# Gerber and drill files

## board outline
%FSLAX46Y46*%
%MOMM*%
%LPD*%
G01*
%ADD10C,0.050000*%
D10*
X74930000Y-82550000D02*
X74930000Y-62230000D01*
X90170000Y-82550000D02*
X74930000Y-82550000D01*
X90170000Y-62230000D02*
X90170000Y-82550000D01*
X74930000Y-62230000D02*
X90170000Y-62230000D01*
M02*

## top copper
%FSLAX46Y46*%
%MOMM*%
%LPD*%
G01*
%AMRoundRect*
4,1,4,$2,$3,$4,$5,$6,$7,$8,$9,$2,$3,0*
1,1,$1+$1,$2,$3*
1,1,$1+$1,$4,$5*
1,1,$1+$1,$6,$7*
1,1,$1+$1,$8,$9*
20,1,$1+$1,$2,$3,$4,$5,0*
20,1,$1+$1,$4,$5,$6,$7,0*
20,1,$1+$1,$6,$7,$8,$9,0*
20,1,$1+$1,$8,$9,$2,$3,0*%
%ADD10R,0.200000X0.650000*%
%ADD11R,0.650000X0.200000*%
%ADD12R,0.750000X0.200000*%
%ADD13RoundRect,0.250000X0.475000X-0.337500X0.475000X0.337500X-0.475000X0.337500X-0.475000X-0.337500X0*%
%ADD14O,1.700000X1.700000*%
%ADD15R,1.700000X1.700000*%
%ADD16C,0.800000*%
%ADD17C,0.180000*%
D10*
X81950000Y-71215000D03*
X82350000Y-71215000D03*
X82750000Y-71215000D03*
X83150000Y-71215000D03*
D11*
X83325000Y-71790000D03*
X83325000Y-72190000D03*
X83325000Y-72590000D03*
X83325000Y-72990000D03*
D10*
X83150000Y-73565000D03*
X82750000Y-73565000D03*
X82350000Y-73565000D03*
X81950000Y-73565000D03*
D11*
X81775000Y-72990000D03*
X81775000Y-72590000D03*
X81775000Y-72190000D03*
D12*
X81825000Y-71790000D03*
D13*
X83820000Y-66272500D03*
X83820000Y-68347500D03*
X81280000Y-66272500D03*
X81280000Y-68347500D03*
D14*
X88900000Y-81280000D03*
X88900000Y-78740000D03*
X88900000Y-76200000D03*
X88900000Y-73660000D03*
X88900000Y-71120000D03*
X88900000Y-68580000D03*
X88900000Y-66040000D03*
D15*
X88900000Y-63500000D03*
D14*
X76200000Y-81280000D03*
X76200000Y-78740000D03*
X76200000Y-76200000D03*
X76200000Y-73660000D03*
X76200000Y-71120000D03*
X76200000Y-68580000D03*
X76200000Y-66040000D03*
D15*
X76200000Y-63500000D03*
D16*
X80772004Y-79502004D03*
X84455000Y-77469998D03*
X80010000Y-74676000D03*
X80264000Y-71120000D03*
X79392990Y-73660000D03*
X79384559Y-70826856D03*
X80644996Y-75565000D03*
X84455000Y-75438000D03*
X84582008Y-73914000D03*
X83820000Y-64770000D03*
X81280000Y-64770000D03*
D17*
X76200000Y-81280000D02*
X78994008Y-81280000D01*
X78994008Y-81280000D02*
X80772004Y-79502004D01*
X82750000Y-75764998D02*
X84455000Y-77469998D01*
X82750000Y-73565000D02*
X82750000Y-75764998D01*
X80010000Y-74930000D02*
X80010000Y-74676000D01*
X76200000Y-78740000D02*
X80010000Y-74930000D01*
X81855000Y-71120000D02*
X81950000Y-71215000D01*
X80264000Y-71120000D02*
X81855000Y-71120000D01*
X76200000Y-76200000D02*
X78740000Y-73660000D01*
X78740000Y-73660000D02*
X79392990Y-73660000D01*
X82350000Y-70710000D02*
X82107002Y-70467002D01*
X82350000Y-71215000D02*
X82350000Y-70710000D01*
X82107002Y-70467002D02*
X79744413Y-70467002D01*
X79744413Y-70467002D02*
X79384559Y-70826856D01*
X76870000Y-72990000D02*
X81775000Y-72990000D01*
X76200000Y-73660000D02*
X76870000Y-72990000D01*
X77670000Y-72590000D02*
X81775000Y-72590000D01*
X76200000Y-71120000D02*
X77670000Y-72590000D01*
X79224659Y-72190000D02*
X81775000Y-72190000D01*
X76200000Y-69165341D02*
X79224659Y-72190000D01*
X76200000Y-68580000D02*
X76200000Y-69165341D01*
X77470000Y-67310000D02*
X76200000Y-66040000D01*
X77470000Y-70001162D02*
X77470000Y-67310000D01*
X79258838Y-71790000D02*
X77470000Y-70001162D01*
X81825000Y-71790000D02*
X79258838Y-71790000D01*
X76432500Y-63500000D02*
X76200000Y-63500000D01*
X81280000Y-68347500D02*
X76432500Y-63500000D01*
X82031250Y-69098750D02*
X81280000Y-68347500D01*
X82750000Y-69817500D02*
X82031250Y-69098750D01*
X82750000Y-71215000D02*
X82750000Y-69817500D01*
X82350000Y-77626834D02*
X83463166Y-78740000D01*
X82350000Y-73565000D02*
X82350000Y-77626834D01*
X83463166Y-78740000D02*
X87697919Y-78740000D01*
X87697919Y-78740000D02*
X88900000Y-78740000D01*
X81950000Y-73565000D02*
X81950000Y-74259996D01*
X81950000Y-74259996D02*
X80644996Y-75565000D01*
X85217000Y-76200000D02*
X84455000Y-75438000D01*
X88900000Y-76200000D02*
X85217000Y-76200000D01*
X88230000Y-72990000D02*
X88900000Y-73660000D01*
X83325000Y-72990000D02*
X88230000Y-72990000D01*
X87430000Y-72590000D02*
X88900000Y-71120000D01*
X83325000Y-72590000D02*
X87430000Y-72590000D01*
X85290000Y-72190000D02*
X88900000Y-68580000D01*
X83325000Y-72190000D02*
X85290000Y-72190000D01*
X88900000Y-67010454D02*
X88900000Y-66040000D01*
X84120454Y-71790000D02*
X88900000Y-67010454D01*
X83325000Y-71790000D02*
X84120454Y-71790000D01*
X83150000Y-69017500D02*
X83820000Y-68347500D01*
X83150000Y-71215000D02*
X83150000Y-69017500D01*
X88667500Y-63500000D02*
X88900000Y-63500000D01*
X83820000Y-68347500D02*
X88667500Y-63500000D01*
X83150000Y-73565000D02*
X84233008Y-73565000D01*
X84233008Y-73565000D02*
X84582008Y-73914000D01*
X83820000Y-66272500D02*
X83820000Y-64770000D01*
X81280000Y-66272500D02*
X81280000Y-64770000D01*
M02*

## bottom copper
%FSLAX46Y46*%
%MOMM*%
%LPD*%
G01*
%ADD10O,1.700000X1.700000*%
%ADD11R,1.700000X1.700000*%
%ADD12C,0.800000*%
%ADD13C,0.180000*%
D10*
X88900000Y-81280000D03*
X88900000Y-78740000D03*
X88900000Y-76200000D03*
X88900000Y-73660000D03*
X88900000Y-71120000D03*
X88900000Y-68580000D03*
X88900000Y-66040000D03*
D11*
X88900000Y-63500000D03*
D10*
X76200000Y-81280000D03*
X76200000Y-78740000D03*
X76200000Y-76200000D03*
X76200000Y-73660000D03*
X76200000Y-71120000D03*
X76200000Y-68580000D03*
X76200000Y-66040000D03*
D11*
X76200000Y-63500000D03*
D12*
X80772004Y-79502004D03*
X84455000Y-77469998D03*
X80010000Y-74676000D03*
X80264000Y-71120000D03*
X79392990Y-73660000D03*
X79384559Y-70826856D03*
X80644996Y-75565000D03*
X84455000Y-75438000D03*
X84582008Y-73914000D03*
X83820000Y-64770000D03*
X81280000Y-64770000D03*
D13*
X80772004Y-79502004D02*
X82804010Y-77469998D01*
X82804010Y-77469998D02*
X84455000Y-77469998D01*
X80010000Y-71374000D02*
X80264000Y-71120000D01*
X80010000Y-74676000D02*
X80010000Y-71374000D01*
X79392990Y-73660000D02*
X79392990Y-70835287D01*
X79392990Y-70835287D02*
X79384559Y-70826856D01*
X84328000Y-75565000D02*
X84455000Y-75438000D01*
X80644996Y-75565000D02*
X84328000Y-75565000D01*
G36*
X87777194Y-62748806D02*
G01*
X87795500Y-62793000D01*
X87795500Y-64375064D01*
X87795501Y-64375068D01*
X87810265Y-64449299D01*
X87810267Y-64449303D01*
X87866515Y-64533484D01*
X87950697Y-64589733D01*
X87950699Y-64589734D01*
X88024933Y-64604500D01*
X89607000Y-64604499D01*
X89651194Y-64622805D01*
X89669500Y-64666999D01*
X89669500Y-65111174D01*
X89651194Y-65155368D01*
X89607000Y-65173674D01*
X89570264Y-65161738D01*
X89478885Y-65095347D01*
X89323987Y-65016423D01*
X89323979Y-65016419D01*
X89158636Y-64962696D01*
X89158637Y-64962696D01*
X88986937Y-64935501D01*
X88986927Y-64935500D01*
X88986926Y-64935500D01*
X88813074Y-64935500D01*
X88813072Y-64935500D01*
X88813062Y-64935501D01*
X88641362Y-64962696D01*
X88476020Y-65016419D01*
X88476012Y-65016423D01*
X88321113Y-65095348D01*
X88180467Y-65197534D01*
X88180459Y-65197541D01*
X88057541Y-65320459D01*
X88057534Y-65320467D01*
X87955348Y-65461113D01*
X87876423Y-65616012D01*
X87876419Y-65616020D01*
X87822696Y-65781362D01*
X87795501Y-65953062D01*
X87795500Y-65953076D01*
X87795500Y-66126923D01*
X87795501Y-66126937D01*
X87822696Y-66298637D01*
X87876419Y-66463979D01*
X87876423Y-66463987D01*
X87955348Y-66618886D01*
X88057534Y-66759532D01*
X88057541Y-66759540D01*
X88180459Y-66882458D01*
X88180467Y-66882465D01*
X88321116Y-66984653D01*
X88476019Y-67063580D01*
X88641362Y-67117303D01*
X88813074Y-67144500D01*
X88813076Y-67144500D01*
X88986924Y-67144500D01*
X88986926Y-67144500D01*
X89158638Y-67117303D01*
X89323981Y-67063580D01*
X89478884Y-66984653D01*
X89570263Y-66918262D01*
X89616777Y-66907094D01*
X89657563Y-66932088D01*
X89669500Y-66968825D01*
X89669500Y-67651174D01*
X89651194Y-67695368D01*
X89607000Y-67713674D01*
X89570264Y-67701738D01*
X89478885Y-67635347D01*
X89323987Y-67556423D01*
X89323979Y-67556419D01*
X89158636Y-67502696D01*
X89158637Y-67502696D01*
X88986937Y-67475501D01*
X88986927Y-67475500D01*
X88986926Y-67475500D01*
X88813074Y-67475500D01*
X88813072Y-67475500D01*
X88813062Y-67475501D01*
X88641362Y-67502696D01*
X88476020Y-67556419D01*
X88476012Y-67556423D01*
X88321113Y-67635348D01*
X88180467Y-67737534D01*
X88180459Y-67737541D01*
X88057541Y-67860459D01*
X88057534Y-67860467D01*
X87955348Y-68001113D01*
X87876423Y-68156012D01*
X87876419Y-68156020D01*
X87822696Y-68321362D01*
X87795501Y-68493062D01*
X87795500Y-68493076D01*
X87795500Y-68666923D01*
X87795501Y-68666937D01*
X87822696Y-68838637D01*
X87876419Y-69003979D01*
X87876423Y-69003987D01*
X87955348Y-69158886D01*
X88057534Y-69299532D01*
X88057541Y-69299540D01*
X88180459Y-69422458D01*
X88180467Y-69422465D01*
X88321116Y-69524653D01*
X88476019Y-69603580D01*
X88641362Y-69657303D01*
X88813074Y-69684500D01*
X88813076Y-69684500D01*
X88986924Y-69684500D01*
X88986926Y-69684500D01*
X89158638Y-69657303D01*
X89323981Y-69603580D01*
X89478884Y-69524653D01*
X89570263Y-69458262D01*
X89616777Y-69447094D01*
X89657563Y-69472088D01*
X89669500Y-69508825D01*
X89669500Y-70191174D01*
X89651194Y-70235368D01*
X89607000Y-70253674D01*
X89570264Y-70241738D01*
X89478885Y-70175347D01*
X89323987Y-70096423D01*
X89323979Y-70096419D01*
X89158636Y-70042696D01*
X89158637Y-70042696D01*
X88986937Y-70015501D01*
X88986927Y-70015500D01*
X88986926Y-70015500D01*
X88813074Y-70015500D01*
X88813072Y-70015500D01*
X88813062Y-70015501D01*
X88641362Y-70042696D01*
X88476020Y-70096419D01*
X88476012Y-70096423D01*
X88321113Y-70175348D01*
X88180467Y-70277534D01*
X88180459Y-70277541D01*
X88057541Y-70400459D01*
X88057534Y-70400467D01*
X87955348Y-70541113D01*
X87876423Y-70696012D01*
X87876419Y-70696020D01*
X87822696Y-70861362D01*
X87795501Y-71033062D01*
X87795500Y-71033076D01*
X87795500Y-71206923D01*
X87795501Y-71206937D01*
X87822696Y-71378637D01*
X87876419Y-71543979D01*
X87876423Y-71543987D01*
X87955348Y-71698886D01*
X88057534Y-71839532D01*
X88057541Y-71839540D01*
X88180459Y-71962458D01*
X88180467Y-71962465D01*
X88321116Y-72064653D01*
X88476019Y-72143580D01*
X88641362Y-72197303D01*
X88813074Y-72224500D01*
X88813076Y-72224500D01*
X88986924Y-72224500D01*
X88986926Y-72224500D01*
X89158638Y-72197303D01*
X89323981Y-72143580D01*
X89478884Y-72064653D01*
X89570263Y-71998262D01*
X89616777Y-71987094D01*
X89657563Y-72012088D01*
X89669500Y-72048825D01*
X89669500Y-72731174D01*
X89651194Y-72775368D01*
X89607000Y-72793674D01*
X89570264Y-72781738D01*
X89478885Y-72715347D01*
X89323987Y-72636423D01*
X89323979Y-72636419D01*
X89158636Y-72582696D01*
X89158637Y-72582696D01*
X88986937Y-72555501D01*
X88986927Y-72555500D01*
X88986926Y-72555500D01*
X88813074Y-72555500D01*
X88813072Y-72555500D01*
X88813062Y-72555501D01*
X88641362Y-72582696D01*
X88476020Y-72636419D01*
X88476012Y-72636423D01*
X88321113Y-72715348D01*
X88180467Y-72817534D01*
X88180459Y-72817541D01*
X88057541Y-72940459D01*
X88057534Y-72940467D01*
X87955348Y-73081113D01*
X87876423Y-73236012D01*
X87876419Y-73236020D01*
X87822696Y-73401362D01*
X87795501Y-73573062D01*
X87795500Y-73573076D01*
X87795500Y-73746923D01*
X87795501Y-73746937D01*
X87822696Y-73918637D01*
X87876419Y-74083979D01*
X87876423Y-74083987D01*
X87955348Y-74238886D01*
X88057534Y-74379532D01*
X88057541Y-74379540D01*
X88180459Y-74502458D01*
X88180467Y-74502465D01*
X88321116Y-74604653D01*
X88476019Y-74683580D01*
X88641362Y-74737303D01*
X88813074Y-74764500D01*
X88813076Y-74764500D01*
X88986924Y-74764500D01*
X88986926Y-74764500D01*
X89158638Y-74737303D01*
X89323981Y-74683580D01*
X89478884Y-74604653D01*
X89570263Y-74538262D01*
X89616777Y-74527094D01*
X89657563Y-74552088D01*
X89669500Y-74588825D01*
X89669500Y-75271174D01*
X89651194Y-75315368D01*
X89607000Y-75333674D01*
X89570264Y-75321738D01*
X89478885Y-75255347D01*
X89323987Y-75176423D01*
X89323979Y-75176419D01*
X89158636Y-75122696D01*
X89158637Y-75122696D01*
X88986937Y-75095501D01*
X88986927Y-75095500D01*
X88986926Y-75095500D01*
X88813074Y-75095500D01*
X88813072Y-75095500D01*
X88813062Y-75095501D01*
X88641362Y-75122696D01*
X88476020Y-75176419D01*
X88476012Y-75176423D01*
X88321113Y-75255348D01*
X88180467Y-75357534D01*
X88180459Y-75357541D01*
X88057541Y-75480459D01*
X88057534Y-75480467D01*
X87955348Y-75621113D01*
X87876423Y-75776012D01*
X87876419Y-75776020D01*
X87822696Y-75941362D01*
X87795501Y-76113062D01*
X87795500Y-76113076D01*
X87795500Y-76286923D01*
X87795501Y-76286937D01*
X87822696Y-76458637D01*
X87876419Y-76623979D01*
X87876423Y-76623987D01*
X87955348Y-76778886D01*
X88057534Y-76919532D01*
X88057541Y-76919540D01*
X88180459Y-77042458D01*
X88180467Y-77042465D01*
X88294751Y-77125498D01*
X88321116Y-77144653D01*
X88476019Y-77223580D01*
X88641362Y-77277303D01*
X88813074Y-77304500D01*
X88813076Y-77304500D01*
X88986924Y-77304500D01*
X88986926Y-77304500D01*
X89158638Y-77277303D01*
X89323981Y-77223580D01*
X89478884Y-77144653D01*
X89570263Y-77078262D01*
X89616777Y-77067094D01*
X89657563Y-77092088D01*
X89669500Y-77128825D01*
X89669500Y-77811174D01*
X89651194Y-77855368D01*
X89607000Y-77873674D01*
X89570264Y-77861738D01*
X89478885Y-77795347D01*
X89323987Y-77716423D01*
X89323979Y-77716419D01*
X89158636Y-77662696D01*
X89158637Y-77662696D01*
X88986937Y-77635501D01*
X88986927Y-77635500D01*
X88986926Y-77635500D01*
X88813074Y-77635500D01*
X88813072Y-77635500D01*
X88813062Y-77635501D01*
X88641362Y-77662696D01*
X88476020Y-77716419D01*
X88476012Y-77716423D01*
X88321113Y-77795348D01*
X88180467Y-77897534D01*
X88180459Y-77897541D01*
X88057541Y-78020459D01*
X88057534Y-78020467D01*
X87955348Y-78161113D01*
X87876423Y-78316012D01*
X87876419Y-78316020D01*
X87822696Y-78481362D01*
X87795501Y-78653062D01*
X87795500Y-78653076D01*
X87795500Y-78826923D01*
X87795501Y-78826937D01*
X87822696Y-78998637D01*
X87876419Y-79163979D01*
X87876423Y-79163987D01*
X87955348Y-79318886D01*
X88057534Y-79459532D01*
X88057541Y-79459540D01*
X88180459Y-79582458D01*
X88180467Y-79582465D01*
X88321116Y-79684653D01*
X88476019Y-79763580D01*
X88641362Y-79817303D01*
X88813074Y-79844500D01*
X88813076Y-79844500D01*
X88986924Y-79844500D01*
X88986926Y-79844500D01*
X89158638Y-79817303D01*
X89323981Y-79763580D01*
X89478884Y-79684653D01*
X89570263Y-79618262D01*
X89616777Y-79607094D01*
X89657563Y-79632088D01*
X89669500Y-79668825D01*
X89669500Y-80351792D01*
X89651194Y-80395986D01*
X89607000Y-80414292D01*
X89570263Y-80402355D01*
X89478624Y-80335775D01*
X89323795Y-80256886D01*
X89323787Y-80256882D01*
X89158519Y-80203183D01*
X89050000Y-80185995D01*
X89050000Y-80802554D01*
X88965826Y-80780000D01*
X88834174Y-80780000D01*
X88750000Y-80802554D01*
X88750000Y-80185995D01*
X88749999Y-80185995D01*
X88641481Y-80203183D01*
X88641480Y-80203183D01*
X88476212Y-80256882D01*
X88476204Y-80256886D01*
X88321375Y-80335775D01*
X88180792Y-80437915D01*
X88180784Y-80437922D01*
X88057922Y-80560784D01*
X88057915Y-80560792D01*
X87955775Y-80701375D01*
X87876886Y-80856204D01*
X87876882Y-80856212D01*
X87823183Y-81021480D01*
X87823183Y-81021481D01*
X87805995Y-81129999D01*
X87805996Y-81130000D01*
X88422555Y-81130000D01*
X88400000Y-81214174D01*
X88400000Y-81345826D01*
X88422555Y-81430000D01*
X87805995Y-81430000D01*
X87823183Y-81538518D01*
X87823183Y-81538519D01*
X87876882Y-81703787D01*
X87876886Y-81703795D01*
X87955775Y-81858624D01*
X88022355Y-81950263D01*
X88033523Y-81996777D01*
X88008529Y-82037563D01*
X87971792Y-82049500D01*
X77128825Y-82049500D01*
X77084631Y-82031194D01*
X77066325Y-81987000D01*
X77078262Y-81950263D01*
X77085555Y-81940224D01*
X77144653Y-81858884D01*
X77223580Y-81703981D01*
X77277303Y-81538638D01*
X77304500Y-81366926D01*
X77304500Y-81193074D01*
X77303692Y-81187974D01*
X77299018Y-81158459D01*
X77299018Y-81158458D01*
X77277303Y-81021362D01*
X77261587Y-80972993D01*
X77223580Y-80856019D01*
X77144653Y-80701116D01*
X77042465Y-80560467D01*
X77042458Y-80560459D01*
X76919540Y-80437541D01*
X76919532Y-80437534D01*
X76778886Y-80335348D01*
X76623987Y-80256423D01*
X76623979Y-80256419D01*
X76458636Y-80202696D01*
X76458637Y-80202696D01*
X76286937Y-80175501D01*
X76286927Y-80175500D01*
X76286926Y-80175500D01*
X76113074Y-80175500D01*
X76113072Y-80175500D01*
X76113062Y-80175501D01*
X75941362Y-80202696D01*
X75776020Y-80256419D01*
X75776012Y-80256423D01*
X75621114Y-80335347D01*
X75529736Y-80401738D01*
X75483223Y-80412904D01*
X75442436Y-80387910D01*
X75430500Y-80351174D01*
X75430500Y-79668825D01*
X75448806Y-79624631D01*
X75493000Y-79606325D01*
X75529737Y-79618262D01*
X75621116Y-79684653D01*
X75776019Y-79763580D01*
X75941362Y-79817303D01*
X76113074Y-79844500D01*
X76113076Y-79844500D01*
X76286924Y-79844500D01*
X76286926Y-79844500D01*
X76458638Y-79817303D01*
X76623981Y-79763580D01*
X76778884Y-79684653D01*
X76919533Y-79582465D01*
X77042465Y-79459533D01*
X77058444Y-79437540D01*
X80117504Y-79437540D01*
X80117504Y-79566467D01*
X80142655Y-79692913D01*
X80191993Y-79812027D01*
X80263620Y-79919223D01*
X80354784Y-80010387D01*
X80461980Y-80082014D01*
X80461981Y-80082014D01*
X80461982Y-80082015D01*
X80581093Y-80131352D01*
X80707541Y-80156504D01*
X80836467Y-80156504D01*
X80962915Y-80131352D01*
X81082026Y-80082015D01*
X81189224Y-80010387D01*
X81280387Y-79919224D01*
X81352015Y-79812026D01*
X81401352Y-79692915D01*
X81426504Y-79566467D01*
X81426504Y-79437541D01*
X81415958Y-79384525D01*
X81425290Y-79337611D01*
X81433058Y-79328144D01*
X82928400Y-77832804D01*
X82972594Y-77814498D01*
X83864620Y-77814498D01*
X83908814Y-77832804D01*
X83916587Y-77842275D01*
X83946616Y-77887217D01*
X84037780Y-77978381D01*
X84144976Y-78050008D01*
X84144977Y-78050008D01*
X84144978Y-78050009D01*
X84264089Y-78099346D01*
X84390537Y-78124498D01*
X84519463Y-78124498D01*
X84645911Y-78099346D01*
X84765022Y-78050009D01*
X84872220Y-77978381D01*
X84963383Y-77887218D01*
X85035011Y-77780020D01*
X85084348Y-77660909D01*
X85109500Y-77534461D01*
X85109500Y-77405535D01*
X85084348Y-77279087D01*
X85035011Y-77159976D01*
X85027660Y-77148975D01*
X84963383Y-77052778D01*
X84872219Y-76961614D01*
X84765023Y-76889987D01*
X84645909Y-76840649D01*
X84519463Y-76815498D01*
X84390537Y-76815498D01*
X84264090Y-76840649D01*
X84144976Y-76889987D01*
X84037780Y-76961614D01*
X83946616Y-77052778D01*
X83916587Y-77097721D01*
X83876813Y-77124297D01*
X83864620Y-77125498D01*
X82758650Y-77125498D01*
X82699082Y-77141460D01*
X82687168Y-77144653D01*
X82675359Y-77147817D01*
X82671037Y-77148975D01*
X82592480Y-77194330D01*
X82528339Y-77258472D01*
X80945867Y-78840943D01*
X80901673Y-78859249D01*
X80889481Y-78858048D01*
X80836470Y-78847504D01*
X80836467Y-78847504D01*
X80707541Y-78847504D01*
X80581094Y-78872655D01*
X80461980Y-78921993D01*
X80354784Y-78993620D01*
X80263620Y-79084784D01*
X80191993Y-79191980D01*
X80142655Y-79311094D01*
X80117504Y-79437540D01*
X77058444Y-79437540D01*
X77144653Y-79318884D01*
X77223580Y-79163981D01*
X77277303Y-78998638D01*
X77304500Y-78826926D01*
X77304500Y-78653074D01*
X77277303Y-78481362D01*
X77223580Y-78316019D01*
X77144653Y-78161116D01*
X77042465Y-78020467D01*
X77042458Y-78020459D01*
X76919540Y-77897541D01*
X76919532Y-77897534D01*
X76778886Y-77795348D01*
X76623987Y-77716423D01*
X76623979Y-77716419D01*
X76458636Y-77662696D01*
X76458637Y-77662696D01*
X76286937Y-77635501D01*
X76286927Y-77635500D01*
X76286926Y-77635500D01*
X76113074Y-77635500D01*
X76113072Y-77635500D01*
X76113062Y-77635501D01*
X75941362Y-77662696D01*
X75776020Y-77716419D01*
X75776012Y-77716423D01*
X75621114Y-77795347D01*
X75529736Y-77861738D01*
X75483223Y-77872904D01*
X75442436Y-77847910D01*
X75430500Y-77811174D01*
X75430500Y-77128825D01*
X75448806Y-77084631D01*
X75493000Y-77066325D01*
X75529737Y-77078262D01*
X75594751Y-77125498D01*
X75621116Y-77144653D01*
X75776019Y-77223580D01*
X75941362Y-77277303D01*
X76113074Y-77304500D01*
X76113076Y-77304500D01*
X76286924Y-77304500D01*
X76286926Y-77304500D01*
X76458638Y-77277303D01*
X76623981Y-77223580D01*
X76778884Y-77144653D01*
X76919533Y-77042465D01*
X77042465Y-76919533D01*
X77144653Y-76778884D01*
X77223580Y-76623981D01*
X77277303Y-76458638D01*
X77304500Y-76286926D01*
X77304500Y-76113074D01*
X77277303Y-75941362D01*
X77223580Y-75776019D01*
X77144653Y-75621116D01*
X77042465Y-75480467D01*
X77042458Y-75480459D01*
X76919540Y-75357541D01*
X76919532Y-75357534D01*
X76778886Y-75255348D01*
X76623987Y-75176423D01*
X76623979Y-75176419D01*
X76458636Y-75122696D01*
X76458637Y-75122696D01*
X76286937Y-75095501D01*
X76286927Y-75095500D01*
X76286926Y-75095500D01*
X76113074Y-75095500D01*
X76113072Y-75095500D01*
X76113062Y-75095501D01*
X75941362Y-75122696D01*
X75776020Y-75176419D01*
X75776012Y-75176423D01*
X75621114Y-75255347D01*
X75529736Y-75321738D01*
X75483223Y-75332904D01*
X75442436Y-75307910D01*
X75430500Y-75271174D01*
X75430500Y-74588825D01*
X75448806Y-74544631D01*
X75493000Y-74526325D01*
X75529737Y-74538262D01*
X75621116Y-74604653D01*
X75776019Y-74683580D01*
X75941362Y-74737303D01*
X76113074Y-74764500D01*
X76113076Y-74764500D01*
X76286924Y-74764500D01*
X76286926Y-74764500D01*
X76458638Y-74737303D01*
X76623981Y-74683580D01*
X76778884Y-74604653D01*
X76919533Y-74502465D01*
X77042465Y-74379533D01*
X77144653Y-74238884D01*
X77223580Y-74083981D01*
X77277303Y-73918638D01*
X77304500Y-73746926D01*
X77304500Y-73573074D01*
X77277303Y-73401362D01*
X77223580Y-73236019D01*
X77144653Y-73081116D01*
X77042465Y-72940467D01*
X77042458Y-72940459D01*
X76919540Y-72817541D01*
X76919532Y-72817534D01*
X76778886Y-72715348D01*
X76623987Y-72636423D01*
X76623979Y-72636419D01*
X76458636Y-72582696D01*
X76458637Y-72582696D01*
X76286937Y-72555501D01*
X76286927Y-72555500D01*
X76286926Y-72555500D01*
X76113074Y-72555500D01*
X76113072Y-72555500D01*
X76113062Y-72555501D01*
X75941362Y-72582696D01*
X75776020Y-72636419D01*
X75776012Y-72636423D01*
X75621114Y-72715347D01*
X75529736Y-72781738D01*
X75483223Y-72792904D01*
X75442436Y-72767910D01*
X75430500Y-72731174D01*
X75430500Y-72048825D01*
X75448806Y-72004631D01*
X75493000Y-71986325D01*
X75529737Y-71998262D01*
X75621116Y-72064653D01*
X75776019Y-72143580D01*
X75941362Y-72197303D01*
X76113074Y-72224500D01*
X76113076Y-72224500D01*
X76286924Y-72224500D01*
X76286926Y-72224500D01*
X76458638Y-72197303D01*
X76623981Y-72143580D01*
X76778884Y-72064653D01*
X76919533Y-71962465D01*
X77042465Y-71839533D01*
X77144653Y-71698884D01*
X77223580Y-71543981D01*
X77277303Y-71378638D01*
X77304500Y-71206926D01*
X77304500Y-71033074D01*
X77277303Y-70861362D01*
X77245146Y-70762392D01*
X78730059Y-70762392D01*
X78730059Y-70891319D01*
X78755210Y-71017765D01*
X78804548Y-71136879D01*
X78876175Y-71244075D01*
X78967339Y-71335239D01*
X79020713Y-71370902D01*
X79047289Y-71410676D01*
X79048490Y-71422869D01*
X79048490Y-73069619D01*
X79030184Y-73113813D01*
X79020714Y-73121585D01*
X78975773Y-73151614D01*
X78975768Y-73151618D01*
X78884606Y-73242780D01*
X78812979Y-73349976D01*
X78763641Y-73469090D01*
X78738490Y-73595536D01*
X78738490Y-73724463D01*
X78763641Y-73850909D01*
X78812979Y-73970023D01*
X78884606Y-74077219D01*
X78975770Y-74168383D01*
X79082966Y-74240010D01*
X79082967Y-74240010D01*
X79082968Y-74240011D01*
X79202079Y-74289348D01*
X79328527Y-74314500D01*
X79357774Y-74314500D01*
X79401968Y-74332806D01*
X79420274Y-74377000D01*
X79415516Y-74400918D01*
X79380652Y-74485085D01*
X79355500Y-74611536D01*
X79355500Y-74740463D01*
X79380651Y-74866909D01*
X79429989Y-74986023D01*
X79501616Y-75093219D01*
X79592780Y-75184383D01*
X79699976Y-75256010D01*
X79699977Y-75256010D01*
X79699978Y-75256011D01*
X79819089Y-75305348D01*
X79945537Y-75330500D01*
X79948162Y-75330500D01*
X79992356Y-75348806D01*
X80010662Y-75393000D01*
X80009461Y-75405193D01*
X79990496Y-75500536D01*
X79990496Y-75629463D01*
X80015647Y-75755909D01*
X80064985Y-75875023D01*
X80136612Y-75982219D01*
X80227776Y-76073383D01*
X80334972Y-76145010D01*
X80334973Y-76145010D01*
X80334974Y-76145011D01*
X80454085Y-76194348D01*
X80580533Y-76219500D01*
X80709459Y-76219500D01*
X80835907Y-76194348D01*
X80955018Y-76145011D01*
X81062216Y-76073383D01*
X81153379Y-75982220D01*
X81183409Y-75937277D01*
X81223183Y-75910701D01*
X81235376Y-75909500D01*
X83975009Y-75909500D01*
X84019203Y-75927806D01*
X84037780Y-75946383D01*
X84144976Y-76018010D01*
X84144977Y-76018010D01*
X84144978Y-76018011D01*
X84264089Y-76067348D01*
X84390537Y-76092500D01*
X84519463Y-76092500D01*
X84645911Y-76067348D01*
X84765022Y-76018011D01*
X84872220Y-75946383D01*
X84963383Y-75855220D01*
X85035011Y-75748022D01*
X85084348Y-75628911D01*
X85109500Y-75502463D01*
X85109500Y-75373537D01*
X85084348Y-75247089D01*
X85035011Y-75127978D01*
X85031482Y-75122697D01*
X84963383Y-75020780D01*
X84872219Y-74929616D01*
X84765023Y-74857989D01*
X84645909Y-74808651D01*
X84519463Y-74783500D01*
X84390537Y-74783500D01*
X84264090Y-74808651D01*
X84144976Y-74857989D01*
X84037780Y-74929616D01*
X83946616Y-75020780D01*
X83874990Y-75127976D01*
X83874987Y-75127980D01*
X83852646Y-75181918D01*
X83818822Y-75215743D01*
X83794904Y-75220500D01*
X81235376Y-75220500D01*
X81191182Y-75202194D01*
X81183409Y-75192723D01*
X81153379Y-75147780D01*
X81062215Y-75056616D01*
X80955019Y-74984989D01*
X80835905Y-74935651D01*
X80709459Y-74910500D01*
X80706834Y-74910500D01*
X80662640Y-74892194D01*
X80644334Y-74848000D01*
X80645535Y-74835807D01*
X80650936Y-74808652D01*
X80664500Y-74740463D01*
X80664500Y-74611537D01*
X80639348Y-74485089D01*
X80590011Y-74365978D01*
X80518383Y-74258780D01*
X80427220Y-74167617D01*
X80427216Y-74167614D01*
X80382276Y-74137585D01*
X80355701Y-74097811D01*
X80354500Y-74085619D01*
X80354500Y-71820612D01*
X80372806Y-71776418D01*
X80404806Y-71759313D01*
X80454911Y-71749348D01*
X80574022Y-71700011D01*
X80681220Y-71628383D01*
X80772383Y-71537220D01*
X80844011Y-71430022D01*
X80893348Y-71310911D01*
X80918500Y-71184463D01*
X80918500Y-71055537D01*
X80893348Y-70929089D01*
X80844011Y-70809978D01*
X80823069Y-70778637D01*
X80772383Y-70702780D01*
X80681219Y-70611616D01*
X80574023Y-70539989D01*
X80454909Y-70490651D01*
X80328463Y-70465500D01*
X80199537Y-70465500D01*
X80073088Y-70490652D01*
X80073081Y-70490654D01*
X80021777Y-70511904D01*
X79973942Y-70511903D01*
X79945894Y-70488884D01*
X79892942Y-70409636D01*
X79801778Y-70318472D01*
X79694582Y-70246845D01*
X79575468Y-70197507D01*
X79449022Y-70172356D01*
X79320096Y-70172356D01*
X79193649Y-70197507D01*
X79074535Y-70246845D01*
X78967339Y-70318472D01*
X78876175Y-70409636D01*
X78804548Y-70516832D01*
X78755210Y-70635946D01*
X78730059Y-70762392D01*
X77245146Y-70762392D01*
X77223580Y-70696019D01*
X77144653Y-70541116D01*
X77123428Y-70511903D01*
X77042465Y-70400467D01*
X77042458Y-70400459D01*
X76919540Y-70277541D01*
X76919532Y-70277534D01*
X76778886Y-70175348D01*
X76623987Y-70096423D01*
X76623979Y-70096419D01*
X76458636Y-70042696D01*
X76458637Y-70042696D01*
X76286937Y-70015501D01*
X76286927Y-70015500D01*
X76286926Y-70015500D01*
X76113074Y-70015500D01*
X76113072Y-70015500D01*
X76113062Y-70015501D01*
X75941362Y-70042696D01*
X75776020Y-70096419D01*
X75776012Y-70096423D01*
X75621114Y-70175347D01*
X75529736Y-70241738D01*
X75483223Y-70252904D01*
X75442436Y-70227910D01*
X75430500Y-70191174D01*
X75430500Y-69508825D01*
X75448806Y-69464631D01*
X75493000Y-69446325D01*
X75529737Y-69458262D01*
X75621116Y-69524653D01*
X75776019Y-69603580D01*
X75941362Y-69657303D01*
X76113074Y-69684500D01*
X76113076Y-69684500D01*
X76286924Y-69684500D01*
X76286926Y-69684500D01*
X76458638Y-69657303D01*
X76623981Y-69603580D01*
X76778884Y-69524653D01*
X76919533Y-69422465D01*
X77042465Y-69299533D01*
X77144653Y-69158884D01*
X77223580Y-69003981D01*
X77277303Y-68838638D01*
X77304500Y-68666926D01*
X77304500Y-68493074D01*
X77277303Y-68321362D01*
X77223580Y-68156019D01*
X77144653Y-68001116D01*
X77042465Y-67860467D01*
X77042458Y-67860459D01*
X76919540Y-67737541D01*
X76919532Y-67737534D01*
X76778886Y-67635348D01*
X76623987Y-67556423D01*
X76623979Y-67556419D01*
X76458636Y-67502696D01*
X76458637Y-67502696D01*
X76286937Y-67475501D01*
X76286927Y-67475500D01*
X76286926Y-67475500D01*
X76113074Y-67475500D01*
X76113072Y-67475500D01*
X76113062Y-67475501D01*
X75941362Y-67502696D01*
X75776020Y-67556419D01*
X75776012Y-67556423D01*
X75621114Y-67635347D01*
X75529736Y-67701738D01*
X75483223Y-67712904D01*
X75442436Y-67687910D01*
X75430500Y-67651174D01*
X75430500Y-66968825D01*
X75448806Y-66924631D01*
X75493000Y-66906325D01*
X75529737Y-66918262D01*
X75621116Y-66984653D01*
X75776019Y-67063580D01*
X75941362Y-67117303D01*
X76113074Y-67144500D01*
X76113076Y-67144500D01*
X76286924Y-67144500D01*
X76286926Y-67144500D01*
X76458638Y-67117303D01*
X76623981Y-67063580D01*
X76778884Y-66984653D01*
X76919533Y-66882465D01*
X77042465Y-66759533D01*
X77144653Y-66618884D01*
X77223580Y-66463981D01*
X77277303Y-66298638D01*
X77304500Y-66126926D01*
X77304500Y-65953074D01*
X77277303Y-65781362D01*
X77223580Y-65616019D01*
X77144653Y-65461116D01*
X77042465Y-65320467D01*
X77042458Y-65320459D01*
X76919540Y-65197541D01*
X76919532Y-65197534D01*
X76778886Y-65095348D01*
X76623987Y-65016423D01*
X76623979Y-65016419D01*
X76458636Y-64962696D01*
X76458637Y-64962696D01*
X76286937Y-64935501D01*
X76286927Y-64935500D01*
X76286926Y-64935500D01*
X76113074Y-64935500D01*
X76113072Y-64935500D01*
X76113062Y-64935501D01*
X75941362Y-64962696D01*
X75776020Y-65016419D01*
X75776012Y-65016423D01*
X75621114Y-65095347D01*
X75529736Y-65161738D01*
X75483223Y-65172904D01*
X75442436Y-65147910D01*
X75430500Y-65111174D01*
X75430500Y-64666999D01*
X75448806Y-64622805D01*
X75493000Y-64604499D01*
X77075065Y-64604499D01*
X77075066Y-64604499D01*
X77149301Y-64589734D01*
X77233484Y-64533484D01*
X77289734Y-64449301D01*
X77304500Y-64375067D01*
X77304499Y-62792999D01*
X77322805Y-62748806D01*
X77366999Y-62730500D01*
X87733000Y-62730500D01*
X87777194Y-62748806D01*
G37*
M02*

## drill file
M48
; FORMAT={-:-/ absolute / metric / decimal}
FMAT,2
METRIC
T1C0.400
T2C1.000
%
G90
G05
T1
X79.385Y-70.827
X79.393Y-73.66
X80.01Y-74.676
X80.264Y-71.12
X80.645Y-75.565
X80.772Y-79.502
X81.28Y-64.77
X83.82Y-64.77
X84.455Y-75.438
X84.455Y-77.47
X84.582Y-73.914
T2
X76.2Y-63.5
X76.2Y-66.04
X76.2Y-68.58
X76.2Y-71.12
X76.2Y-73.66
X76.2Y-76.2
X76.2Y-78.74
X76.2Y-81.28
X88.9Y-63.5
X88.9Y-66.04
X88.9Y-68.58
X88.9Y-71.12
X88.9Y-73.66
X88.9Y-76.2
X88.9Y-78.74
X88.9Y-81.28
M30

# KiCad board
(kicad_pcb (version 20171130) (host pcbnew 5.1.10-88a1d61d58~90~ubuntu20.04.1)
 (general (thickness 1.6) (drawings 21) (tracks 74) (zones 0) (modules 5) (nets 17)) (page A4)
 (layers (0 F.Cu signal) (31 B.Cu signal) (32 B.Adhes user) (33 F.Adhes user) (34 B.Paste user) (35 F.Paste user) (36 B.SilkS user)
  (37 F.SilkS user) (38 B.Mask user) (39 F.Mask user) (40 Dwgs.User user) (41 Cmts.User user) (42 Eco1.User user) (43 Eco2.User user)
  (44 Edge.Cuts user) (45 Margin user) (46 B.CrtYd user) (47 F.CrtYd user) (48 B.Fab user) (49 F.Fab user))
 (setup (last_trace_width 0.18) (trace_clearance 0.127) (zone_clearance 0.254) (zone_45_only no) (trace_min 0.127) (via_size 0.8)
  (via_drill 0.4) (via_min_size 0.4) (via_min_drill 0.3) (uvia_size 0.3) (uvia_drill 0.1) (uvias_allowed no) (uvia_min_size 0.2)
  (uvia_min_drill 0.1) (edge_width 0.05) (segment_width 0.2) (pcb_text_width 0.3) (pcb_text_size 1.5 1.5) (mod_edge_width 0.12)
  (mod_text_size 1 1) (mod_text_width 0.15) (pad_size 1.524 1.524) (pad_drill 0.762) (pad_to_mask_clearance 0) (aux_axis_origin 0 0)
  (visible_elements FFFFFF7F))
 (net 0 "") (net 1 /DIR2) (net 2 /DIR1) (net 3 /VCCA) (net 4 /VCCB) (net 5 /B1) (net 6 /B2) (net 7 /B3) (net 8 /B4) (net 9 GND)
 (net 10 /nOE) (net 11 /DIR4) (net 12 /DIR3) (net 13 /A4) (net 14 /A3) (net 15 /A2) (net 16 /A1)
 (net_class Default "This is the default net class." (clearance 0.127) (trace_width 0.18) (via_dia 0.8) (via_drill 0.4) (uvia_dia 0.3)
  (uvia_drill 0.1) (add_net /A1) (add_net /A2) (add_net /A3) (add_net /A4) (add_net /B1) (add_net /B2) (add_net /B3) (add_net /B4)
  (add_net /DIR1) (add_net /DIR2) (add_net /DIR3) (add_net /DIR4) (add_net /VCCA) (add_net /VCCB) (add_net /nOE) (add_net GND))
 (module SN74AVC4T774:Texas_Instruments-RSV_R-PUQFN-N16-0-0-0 (layer F.Cu) (at 82.55 72.39 270)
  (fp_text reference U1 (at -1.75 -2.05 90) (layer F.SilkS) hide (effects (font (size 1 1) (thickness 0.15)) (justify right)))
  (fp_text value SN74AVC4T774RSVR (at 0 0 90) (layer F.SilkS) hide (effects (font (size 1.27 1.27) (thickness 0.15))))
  (pad 16 smd rect (at -1.175 0.6 270) (size 0.65 0.2) (layers F.Cu F.Paste F.Mask) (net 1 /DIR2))
  (pad 15 smd rect (at -1.175 0.2 270) (size 0.65 0.2) (layers F.Cu F.Paste F.Mask) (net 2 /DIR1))
  (pad 14 smd rect (at -1.175 -0.2 270) (size 0.65 0.2) (layers F.Cu F.Paste F.Mask) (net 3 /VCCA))
  (pad 13 smd rect (at -1.175 -0.6 270) (size 0.65 0.2) (layers F.Cu F.Paste F.Mask) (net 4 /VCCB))
  (pad 12 smd rect (at -0.6 -0.775 270) (size 0.2 0.65) (layers F.Cu F.Paste F.Mask) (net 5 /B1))
  (pad 11 smd rect (at -0.2 -0.775 270) (size 0.2 0.65) (layers F.Cu F.Paste F.Mask) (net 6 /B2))
  (pad 10 smd rect (at 0.2 -0.775 270) (size 0.2 0.65) (layers F.Cu F.Paste F.Mask) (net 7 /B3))
  (pad 9 smd rect (at 0.6 -0.775 270) (size 0.2 0.65) (layers F.Cu F.Paste F.Mask) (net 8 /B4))
  (pad 8 smd rect (at 1.175 -0.6 270) (size 0.65 0.2) (layers F.Cu F.Paste F.Mask) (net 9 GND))
  (pad 7 smd rect (at 1.175 -0.2 270) (size 0.65 0.2) (layers F.Cu F.Paste F.Mask) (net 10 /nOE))
  (pad 6 smd rect (at 1.175 0.2 270) (size 0.65 0.2) (layers F.Cu F.Paste F.Mask) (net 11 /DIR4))
  (pad 5 smd rect (at 1.175 0.6 270) (size 0.65 0.2) (layers F.Cu F.Paste F.Mask) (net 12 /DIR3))
  (pad 4 smd rect (at 0.6 0.775 270) (size 0.2 0.65) (layers F.Cu F.Paste F.Mask) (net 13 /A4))
  (pad 3 smd rect (at 0.2 0.775 270) (size 0.2 0.65) (layers F.Cu F.Paste F.Mask) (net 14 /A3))
  (pad 2 smd rect (at -0.2 0.775 270) (size 0.2 0.65) (layers F.Cu F.Paste F.Mask) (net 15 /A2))
  (pad 1 smd rect (at -0.6 0.725 270) (size 0.2 0.75) (layers F.Cu F.Paste F.Mask) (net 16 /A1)))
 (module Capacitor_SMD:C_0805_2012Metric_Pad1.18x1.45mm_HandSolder (layer F.Cu) (at 83.82 67.31 90)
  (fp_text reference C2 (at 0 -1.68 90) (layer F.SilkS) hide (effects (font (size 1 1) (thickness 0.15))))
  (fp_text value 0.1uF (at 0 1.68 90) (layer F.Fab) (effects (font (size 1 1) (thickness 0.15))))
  (pad 2 smd roundrect (at 1.0375 0 90) (size 1.175 1.45) (layers F.Cu F.Paste F.Mask) (roundrect_rratio 0.212766) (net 9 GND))
  (pad 1 smd roundrect (at -1.0375 0 90) (size 1.175 1.45) (layers F.Cu F.Paste F.Mask) (roundrect_rratio 0.212766) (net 4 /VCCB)))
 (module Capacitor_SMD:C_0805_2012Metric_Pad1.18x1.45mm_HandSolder (layer F.Cu) (at 81.28 67.31 90)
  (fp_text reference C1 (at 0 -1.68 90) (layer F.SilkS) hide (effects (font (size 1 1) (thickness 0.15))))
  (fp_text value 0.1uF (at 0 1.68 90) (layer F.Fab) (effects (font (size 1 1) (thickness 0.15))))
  (pad 2 smd roundrect (at 1.0375 0 90) (size 1.175 1.45) (layers F.Cu F.Paste F.Mask) (roundrect_rratio 0.212766) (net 9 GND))
  (pad 1 smd roundrect (at -1.0375 0 90) (size 1.175 1.45) (layers F.Cu F.Paste F.Mask) (roundrect_rratio 0.212766) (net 3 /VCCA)))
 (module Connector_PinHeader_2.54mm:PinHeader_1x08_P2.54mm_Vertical (layer B.Cu) (at 88.9 63.5 180)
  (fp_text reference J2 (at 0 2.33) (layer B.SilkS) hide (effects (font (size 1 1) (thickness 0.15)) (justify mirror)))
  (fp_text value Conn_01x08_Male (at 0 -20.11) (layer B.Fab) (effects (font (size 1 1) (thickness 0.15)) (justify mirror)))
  (pad 8 thru_hole oval (at 0 -17.78 180) (size 1.7 1.7) (drill 1) (layers *.Cu *.Mask) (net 9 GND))
  (pad 7 thru_hole oval (at 0 -15.24 180) (size 1.7 1.7) (drill 1) (layers *.Cu *.Mask) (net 11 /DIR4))
  (pad 6 thru_hole oval (at 0 -12.7 180) (size 1.7 1.7) (drill 1) (layers *.Cu *.Mask) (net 12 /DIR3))
  (pad 5 thru_hole oval (at 0 -10.16 180) (size 1.7 1.7) (drill 1) (layers *.Cu *.Mask) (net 8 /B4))
  (pad 4 thru_hole oval (at 0 -7.62 180) (size 1.7 1.7) (drill 1) (layers *.Cu *.Mask) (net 7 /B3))
  (pad 3 thru_hole oval (at 0 -5.08 180) (size 1.7 1.7) (drill 1) (layers *.Cu *.Mask) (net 6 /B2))
  (pad 2 thru_hole oval (at 0 -2.54 180) (size 1.7 1.7) (drill 1) (layers *.Cu *.Mask) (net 5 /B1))
  (pad 1 thru_hole rect (at 0 0 180) (size 1.7 1.7) (drill 1) (layers *.Cu *.Mask) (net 4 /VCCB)))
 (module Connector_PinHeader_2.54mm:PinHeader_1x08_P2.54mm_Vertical (layer B.Cu) (at 76.2 63.5 180)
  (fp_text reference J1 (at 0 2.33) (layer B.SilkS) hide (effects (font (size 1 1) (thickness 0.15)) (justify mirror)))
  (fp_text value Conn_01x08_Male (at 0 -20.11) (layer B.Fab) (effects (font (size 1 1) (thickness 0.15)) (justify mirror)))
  (pad 8 thru_hole oval (at 0 -17.78 180) (size 1.7 1.7) (drill 1) (layers *.Cu *.Mask) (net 10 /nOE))
  (pad 7 thru_hole oval (at 0 -15.24 180) (size 1.7 1.7) (drill 1) (layers *.Cu *.Mask) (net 1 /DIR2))
  (pad 6 thru_hole oval (at 0 -12.7 180) (size 1.7 1.7) (drill 1) (layers *.Cu *.Mask) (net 2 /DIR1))
  (pad 5 thru_hole oval (at 0 -10.16 180) (size 1.7 1.7) (drill 1) (layers *.Cu *.Mask) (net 13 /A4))
  (pad 4 thru_hole oval (at 0 -7.62 180) (size 1.7 1.7) (drill 1) (layers *.Cu *.Mask) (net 14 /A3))
  (pad 3 thru_hole oval (at 0 -5.08 180) (size 1.7 1.7) (drill 1) (layers *.Cu *.Mask) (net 15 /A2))
  (pad 2 thru_hole oval (at 0 -2.54 180) (size 1.7 1.7) (drill 1) (layers *.Cu *.Mask) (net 16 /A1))
  (pad 1 thru_hole rect (at 0 0 180) (size 1.7 1.7) (drill 1) (layers *.Cu *.Mask) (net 3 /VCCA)))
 (gr_line (start 74.93 82.55) (end 74.93 62.23) (layer Edge.Cuts) (width 0.05))
 (gr_line (start 90.17 82.55) (end 74.93 82.55) (layer Edge.Cuts) (width 0.05))
 (gr_line (start 90.17 62.23) (end 90.17 82.55) (layer Edge.Cuts) (width 0.05))
 (gr_line (start 74.93 62.23) (end 90.17 62.23) (layer Edge.Cuts) (width 0.05))
 (via (at 80.772004 79.502004) (size 0.8) (drill 0.4) (layers F.Cu B.Cu) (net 10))
 (segment (start 76.2 81.28) (end 78.994008 81.28) (width 0.18) (layer F.Cu) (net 10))
 (segment (start 78.994008 81.28) (end 80.772004 79.502004) (width 0.18) (layer F.Cu) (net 10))
 (via (at 84.455 77.469998) (size 0.8) (drill 0.4) (layers F.Cu B.Cu) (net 10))
 (segment (start 82.75 75.764998) (end 84.455 77.469998) (width 0.18) (layer F.Cu) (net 10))
 (segment (start 82.75 73.565) (end 82.75 75.764998) (width 0.18) (layer F.Cu) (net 10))
 (segment (start 80.772004 79.502004) (end 82.80401 77.469998) (width 0.18) (layer B.Cu) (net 10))
 (segment (start 82.80401 77.469998) (end 84.455 77.469998) (width 0.18) (layer B.Cu) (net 10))
 (via (at 80.01 74.676) (size 0.8) (drill 0.4) (layers F.Cu B.Cu) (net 1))
 (segment (start 80.01 74.93) (end 80.01 74.676) (width 0.18) (layer F.Cu) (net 1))
 (segment (start 76.2 78.74) (end 80.01 74.93) (width 0.18) (layer F.Cu) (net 1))
 (segment (start 80.01 71.374) (end 80.264 71.12) (width 0.18) (layer B.Cu) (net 1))
 (via (at 80.264 71.12) (size 0.8) (drill 0.4) (layers F.Cu B.Cu) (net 1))
 (segment (start 80.01 74.676) (end 80.01 71.374) (width 0.18) (layer B.Cu) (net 1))
 (segment (start 81.855 71.12) (end 81.95 71.215) (width 0.18) (layer F.Cu) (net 1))
 (segment (start 80.264 71.12) (end 81.855 71.12) (width 0.18) (layer F.Cu) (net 1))
 (via (at 79.39299 73.66) (size 0.8) (drill 0.4) (layers F.Cu B.Cu) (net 2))
 (via (at 79.384559 70.826856) (size 0.8) (drill 0.4) (layers F.Cu B.Cu) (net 2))
 (segment (start 76.2 76.2) (end 78.74 73.66) (width 0.18) (layer F.Cu) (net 2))
 (segment (start 78.74 73.66) (end 79.39299 73.66) (width 0.18) (layer F.Cu) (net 2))
 (segment (start 79.39299 73.66) (end 79.39299 70.835287) (width 0.18) (layer B.Cu) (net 2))
 (segment (start 79.39299 70.835287) (end 79.384559 70.826856) (width 0.18) (layer B.Cu) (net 2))
 (segment (start 82.35 70.71) (end 82.107002 70.467002) (width 0.18) (layer F.Cu) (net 2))
 (segment (start 82.35 71.215) (end 82.35 70.71) (width 0.18) (layer F.Cu) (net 2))
 (segment (start 82.107002 70.467002) (end 79.744413 70.467002) (width 0.18) (layer F.Cu) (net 2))
 (segment (start 79.744413 70.467002) (end 79.384559 70.826856) (width 0.18) (layer F.Cu) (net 2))
 (segment (start 76.87 72.99) (end 81.775 72.99) (width 0.18) (layer F.Cu) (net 13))
 (segment (start 76.2 73.66) (end 76.87 72.99) (width 0.18) (layer F.Cu) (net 13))
 (segment (start 77.67 72.59) (end 81.775 72.59) (width 0.18) (layer F.Cu) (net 14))
 (segment (start 76.2 71.12) (end 77.67 72.59) (width 0.18) (layer F.Cu) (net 14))
 (segment (start 79.224659 72.19) (end 81.775 72.19) (width 0.18) (layer F.Cu) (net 15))
 (segment (start 76.2 69.165341) (end 79.224659 72.19) (width 0.18) (layer F.Cu) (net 15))
 (segment (start 76.2 68.58) (end 76.2 69.165341) (width 0.18) (layer F.Cu) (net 15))
 (segment (start 77.47 67.31) (end 76.2 66.04) (width 0.18) (layer F.Cu) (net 16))
 (segment (start 77.47 70.001162) (end 77.47 67.31) (width 0.18) (layer F.Cu) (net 16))
 (segment (start 79.258838 71.79) (end 77.47 70.001162) (width 0.18) (layer F.Cu) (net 16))
 (segment (start 81.825 71.79) (end 79.258838 71.79) (width 0.18) (layer F.Cu) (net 16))
 (segment (start 76.4325 63.5) (end 76.2 63.5) (width 0.18) (layer F.Cu) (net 3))
 (segment (start 81.28 68.3475) (end 76.4325 63.5) (width 0.18) (layer F.Cu) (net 3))
 (segment (start 82.03125 69.09875) (end 81.28 68.3475) (width 0.18) (layer F.Cu) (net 3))
 (segment (start 82.75 69.8175) (end 82.03125 69.09875) (width 0.18) (layer F.Cu) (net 3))
 (segment (start 82.75 71.215) (end 82.75 69.8175) (width 0.18) (layer F.Cu) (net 3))
 (segment (start 82.35 77.626834) (end 83.463166 78.74) (width 0.18) (layer F.Cu) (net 11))
 (segment (start 82.35 73.565) (end 82.35 77.626834) (width 0.18) (layer F.Cu) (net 11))
 (segment (start 83.463166 78.74) (end 87.697919 78.74) (width 0.18) (layer F.Cu) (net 11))
 (segment (start 87.697919 78.74) (end 88.9 78.74) (width 0.18) (layer F.Cu) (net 11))
 (via (at 80.644996 75.565) (size 0.8) (drill 0.4) (layers F.Cu B.Cu) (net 12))
 (segment (start 81.95 73.565) (end 81.95 74.259996) (width 0.18) (layer F.Cu) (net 12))
 (segment (start 81.95 74.259996) (end 80.644996 75.565) (width 0.18) (layer F.Cu) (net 12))
 (segment (start 84.328 75.565) (end 84.455 75.438) (width 0.18) (layer B.Cu) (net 12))
 (segment (start 80.644996 75.565) (end 84.328 75.565) (width 0.18) (layer B.Cu) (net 12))
 (segment (start 85.217 76.2) (end 84.455 75.438) (width 0.18) (layer F.Cu) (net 12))
 (segment (start 88.9 76.2) (end 85.217 76.2) (width 0.18) (layer F.Cu) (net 12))
 (via (at 84.455 75.438) (size 0.8) (drill 0.4) (layers F.Cu B.Cu) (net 12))
 (segment (start 88.23 72.99) (end 88.9 73.66) (width 0.18) (layer F.Cu) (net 8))
 (segment (start 83.325 72.99) (end 88.23 72.99) (width 0.18) (layer F.Cu) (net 8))
 (segment (start 87.43 72.59) (end 88.9 71.12) (width 0.18) (layer F.Cu) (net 7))
 (segment (start 83.325 72.59) (end 87.43 72.59) (width 0.18) (layer F.Cu) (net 7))
 (segment (start 85.29 72.19) (end 88.9 68.58) (width 0.18) (layer F.Cu) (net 6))
 (segment (start 83.325 72.19) (end 85.29 72.19) (width 0.18) (layer F.Cu) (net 6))
 (segment (start 88.9 67.010454) (end 88.9 66.04) (width 0.18) (layer F.Cu) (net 5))
 (segment (start 84.120454 71.79) (end 88.9 67.010454) (width 0.18) (layer F.Cu) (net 5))
 (segment (start 83.325 71.79) (end 84.120454 71.79) (width 0.18) (layer F.Cu) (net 5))
 (segment (start 83.15 69.0175) (end 83.82 68.3475) (width 0.18) (layer F.Cu) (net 4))
 (segment (start 83.15 71.215) (end 83.15 69.0175) (width 0.18) (layer F.Cu) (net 4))
 (segment (start 88.6675 63.5) (end 88.9 63.5) (width 0.18) (layer F.Cu) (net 4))
 (segment (start 83.82 68.3475) (end 88.6675 63.5) (width 0.18) (layer F.Cu) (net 4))
 (via (at 84.582008 73.914) (size 0.8) (drill 0.4) (layers F.Cu B.Cu) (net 9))
 (segment (start 83.15 73.565) (end 84.233008 73.565) (width 0.18) (layer F.Cu) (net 9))
 (segment (start 84.233008 73.565) (end 84.582008 73.914) (width 0.18) (layer F.Cu) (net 9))
 (via (at 83.82 64.77) (size 0.8) (drill 0.4) (layers F.Cu B.Cu) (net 9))
 (segment (start 83.82 66.2725) (end 83.82 64.77) (width 0.18) (layer F.Cu) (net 9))
 (via (at 81.28 64.77) (size 0.8) (drill 0.4) (layers F.Cu B.Cu) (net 9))
 (segment (start 81.28 66.2725) (end 81.28 64.77) (width 0.18) (layer F.Cu) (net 9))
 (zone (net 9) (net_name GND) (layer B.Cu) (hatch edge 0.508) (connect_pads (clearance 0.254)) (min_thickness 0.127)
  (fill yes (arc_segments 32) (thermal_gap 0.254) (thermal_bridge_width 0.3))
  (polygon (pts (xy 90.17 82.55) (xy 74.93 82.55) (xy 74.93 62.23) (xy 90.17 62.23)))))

